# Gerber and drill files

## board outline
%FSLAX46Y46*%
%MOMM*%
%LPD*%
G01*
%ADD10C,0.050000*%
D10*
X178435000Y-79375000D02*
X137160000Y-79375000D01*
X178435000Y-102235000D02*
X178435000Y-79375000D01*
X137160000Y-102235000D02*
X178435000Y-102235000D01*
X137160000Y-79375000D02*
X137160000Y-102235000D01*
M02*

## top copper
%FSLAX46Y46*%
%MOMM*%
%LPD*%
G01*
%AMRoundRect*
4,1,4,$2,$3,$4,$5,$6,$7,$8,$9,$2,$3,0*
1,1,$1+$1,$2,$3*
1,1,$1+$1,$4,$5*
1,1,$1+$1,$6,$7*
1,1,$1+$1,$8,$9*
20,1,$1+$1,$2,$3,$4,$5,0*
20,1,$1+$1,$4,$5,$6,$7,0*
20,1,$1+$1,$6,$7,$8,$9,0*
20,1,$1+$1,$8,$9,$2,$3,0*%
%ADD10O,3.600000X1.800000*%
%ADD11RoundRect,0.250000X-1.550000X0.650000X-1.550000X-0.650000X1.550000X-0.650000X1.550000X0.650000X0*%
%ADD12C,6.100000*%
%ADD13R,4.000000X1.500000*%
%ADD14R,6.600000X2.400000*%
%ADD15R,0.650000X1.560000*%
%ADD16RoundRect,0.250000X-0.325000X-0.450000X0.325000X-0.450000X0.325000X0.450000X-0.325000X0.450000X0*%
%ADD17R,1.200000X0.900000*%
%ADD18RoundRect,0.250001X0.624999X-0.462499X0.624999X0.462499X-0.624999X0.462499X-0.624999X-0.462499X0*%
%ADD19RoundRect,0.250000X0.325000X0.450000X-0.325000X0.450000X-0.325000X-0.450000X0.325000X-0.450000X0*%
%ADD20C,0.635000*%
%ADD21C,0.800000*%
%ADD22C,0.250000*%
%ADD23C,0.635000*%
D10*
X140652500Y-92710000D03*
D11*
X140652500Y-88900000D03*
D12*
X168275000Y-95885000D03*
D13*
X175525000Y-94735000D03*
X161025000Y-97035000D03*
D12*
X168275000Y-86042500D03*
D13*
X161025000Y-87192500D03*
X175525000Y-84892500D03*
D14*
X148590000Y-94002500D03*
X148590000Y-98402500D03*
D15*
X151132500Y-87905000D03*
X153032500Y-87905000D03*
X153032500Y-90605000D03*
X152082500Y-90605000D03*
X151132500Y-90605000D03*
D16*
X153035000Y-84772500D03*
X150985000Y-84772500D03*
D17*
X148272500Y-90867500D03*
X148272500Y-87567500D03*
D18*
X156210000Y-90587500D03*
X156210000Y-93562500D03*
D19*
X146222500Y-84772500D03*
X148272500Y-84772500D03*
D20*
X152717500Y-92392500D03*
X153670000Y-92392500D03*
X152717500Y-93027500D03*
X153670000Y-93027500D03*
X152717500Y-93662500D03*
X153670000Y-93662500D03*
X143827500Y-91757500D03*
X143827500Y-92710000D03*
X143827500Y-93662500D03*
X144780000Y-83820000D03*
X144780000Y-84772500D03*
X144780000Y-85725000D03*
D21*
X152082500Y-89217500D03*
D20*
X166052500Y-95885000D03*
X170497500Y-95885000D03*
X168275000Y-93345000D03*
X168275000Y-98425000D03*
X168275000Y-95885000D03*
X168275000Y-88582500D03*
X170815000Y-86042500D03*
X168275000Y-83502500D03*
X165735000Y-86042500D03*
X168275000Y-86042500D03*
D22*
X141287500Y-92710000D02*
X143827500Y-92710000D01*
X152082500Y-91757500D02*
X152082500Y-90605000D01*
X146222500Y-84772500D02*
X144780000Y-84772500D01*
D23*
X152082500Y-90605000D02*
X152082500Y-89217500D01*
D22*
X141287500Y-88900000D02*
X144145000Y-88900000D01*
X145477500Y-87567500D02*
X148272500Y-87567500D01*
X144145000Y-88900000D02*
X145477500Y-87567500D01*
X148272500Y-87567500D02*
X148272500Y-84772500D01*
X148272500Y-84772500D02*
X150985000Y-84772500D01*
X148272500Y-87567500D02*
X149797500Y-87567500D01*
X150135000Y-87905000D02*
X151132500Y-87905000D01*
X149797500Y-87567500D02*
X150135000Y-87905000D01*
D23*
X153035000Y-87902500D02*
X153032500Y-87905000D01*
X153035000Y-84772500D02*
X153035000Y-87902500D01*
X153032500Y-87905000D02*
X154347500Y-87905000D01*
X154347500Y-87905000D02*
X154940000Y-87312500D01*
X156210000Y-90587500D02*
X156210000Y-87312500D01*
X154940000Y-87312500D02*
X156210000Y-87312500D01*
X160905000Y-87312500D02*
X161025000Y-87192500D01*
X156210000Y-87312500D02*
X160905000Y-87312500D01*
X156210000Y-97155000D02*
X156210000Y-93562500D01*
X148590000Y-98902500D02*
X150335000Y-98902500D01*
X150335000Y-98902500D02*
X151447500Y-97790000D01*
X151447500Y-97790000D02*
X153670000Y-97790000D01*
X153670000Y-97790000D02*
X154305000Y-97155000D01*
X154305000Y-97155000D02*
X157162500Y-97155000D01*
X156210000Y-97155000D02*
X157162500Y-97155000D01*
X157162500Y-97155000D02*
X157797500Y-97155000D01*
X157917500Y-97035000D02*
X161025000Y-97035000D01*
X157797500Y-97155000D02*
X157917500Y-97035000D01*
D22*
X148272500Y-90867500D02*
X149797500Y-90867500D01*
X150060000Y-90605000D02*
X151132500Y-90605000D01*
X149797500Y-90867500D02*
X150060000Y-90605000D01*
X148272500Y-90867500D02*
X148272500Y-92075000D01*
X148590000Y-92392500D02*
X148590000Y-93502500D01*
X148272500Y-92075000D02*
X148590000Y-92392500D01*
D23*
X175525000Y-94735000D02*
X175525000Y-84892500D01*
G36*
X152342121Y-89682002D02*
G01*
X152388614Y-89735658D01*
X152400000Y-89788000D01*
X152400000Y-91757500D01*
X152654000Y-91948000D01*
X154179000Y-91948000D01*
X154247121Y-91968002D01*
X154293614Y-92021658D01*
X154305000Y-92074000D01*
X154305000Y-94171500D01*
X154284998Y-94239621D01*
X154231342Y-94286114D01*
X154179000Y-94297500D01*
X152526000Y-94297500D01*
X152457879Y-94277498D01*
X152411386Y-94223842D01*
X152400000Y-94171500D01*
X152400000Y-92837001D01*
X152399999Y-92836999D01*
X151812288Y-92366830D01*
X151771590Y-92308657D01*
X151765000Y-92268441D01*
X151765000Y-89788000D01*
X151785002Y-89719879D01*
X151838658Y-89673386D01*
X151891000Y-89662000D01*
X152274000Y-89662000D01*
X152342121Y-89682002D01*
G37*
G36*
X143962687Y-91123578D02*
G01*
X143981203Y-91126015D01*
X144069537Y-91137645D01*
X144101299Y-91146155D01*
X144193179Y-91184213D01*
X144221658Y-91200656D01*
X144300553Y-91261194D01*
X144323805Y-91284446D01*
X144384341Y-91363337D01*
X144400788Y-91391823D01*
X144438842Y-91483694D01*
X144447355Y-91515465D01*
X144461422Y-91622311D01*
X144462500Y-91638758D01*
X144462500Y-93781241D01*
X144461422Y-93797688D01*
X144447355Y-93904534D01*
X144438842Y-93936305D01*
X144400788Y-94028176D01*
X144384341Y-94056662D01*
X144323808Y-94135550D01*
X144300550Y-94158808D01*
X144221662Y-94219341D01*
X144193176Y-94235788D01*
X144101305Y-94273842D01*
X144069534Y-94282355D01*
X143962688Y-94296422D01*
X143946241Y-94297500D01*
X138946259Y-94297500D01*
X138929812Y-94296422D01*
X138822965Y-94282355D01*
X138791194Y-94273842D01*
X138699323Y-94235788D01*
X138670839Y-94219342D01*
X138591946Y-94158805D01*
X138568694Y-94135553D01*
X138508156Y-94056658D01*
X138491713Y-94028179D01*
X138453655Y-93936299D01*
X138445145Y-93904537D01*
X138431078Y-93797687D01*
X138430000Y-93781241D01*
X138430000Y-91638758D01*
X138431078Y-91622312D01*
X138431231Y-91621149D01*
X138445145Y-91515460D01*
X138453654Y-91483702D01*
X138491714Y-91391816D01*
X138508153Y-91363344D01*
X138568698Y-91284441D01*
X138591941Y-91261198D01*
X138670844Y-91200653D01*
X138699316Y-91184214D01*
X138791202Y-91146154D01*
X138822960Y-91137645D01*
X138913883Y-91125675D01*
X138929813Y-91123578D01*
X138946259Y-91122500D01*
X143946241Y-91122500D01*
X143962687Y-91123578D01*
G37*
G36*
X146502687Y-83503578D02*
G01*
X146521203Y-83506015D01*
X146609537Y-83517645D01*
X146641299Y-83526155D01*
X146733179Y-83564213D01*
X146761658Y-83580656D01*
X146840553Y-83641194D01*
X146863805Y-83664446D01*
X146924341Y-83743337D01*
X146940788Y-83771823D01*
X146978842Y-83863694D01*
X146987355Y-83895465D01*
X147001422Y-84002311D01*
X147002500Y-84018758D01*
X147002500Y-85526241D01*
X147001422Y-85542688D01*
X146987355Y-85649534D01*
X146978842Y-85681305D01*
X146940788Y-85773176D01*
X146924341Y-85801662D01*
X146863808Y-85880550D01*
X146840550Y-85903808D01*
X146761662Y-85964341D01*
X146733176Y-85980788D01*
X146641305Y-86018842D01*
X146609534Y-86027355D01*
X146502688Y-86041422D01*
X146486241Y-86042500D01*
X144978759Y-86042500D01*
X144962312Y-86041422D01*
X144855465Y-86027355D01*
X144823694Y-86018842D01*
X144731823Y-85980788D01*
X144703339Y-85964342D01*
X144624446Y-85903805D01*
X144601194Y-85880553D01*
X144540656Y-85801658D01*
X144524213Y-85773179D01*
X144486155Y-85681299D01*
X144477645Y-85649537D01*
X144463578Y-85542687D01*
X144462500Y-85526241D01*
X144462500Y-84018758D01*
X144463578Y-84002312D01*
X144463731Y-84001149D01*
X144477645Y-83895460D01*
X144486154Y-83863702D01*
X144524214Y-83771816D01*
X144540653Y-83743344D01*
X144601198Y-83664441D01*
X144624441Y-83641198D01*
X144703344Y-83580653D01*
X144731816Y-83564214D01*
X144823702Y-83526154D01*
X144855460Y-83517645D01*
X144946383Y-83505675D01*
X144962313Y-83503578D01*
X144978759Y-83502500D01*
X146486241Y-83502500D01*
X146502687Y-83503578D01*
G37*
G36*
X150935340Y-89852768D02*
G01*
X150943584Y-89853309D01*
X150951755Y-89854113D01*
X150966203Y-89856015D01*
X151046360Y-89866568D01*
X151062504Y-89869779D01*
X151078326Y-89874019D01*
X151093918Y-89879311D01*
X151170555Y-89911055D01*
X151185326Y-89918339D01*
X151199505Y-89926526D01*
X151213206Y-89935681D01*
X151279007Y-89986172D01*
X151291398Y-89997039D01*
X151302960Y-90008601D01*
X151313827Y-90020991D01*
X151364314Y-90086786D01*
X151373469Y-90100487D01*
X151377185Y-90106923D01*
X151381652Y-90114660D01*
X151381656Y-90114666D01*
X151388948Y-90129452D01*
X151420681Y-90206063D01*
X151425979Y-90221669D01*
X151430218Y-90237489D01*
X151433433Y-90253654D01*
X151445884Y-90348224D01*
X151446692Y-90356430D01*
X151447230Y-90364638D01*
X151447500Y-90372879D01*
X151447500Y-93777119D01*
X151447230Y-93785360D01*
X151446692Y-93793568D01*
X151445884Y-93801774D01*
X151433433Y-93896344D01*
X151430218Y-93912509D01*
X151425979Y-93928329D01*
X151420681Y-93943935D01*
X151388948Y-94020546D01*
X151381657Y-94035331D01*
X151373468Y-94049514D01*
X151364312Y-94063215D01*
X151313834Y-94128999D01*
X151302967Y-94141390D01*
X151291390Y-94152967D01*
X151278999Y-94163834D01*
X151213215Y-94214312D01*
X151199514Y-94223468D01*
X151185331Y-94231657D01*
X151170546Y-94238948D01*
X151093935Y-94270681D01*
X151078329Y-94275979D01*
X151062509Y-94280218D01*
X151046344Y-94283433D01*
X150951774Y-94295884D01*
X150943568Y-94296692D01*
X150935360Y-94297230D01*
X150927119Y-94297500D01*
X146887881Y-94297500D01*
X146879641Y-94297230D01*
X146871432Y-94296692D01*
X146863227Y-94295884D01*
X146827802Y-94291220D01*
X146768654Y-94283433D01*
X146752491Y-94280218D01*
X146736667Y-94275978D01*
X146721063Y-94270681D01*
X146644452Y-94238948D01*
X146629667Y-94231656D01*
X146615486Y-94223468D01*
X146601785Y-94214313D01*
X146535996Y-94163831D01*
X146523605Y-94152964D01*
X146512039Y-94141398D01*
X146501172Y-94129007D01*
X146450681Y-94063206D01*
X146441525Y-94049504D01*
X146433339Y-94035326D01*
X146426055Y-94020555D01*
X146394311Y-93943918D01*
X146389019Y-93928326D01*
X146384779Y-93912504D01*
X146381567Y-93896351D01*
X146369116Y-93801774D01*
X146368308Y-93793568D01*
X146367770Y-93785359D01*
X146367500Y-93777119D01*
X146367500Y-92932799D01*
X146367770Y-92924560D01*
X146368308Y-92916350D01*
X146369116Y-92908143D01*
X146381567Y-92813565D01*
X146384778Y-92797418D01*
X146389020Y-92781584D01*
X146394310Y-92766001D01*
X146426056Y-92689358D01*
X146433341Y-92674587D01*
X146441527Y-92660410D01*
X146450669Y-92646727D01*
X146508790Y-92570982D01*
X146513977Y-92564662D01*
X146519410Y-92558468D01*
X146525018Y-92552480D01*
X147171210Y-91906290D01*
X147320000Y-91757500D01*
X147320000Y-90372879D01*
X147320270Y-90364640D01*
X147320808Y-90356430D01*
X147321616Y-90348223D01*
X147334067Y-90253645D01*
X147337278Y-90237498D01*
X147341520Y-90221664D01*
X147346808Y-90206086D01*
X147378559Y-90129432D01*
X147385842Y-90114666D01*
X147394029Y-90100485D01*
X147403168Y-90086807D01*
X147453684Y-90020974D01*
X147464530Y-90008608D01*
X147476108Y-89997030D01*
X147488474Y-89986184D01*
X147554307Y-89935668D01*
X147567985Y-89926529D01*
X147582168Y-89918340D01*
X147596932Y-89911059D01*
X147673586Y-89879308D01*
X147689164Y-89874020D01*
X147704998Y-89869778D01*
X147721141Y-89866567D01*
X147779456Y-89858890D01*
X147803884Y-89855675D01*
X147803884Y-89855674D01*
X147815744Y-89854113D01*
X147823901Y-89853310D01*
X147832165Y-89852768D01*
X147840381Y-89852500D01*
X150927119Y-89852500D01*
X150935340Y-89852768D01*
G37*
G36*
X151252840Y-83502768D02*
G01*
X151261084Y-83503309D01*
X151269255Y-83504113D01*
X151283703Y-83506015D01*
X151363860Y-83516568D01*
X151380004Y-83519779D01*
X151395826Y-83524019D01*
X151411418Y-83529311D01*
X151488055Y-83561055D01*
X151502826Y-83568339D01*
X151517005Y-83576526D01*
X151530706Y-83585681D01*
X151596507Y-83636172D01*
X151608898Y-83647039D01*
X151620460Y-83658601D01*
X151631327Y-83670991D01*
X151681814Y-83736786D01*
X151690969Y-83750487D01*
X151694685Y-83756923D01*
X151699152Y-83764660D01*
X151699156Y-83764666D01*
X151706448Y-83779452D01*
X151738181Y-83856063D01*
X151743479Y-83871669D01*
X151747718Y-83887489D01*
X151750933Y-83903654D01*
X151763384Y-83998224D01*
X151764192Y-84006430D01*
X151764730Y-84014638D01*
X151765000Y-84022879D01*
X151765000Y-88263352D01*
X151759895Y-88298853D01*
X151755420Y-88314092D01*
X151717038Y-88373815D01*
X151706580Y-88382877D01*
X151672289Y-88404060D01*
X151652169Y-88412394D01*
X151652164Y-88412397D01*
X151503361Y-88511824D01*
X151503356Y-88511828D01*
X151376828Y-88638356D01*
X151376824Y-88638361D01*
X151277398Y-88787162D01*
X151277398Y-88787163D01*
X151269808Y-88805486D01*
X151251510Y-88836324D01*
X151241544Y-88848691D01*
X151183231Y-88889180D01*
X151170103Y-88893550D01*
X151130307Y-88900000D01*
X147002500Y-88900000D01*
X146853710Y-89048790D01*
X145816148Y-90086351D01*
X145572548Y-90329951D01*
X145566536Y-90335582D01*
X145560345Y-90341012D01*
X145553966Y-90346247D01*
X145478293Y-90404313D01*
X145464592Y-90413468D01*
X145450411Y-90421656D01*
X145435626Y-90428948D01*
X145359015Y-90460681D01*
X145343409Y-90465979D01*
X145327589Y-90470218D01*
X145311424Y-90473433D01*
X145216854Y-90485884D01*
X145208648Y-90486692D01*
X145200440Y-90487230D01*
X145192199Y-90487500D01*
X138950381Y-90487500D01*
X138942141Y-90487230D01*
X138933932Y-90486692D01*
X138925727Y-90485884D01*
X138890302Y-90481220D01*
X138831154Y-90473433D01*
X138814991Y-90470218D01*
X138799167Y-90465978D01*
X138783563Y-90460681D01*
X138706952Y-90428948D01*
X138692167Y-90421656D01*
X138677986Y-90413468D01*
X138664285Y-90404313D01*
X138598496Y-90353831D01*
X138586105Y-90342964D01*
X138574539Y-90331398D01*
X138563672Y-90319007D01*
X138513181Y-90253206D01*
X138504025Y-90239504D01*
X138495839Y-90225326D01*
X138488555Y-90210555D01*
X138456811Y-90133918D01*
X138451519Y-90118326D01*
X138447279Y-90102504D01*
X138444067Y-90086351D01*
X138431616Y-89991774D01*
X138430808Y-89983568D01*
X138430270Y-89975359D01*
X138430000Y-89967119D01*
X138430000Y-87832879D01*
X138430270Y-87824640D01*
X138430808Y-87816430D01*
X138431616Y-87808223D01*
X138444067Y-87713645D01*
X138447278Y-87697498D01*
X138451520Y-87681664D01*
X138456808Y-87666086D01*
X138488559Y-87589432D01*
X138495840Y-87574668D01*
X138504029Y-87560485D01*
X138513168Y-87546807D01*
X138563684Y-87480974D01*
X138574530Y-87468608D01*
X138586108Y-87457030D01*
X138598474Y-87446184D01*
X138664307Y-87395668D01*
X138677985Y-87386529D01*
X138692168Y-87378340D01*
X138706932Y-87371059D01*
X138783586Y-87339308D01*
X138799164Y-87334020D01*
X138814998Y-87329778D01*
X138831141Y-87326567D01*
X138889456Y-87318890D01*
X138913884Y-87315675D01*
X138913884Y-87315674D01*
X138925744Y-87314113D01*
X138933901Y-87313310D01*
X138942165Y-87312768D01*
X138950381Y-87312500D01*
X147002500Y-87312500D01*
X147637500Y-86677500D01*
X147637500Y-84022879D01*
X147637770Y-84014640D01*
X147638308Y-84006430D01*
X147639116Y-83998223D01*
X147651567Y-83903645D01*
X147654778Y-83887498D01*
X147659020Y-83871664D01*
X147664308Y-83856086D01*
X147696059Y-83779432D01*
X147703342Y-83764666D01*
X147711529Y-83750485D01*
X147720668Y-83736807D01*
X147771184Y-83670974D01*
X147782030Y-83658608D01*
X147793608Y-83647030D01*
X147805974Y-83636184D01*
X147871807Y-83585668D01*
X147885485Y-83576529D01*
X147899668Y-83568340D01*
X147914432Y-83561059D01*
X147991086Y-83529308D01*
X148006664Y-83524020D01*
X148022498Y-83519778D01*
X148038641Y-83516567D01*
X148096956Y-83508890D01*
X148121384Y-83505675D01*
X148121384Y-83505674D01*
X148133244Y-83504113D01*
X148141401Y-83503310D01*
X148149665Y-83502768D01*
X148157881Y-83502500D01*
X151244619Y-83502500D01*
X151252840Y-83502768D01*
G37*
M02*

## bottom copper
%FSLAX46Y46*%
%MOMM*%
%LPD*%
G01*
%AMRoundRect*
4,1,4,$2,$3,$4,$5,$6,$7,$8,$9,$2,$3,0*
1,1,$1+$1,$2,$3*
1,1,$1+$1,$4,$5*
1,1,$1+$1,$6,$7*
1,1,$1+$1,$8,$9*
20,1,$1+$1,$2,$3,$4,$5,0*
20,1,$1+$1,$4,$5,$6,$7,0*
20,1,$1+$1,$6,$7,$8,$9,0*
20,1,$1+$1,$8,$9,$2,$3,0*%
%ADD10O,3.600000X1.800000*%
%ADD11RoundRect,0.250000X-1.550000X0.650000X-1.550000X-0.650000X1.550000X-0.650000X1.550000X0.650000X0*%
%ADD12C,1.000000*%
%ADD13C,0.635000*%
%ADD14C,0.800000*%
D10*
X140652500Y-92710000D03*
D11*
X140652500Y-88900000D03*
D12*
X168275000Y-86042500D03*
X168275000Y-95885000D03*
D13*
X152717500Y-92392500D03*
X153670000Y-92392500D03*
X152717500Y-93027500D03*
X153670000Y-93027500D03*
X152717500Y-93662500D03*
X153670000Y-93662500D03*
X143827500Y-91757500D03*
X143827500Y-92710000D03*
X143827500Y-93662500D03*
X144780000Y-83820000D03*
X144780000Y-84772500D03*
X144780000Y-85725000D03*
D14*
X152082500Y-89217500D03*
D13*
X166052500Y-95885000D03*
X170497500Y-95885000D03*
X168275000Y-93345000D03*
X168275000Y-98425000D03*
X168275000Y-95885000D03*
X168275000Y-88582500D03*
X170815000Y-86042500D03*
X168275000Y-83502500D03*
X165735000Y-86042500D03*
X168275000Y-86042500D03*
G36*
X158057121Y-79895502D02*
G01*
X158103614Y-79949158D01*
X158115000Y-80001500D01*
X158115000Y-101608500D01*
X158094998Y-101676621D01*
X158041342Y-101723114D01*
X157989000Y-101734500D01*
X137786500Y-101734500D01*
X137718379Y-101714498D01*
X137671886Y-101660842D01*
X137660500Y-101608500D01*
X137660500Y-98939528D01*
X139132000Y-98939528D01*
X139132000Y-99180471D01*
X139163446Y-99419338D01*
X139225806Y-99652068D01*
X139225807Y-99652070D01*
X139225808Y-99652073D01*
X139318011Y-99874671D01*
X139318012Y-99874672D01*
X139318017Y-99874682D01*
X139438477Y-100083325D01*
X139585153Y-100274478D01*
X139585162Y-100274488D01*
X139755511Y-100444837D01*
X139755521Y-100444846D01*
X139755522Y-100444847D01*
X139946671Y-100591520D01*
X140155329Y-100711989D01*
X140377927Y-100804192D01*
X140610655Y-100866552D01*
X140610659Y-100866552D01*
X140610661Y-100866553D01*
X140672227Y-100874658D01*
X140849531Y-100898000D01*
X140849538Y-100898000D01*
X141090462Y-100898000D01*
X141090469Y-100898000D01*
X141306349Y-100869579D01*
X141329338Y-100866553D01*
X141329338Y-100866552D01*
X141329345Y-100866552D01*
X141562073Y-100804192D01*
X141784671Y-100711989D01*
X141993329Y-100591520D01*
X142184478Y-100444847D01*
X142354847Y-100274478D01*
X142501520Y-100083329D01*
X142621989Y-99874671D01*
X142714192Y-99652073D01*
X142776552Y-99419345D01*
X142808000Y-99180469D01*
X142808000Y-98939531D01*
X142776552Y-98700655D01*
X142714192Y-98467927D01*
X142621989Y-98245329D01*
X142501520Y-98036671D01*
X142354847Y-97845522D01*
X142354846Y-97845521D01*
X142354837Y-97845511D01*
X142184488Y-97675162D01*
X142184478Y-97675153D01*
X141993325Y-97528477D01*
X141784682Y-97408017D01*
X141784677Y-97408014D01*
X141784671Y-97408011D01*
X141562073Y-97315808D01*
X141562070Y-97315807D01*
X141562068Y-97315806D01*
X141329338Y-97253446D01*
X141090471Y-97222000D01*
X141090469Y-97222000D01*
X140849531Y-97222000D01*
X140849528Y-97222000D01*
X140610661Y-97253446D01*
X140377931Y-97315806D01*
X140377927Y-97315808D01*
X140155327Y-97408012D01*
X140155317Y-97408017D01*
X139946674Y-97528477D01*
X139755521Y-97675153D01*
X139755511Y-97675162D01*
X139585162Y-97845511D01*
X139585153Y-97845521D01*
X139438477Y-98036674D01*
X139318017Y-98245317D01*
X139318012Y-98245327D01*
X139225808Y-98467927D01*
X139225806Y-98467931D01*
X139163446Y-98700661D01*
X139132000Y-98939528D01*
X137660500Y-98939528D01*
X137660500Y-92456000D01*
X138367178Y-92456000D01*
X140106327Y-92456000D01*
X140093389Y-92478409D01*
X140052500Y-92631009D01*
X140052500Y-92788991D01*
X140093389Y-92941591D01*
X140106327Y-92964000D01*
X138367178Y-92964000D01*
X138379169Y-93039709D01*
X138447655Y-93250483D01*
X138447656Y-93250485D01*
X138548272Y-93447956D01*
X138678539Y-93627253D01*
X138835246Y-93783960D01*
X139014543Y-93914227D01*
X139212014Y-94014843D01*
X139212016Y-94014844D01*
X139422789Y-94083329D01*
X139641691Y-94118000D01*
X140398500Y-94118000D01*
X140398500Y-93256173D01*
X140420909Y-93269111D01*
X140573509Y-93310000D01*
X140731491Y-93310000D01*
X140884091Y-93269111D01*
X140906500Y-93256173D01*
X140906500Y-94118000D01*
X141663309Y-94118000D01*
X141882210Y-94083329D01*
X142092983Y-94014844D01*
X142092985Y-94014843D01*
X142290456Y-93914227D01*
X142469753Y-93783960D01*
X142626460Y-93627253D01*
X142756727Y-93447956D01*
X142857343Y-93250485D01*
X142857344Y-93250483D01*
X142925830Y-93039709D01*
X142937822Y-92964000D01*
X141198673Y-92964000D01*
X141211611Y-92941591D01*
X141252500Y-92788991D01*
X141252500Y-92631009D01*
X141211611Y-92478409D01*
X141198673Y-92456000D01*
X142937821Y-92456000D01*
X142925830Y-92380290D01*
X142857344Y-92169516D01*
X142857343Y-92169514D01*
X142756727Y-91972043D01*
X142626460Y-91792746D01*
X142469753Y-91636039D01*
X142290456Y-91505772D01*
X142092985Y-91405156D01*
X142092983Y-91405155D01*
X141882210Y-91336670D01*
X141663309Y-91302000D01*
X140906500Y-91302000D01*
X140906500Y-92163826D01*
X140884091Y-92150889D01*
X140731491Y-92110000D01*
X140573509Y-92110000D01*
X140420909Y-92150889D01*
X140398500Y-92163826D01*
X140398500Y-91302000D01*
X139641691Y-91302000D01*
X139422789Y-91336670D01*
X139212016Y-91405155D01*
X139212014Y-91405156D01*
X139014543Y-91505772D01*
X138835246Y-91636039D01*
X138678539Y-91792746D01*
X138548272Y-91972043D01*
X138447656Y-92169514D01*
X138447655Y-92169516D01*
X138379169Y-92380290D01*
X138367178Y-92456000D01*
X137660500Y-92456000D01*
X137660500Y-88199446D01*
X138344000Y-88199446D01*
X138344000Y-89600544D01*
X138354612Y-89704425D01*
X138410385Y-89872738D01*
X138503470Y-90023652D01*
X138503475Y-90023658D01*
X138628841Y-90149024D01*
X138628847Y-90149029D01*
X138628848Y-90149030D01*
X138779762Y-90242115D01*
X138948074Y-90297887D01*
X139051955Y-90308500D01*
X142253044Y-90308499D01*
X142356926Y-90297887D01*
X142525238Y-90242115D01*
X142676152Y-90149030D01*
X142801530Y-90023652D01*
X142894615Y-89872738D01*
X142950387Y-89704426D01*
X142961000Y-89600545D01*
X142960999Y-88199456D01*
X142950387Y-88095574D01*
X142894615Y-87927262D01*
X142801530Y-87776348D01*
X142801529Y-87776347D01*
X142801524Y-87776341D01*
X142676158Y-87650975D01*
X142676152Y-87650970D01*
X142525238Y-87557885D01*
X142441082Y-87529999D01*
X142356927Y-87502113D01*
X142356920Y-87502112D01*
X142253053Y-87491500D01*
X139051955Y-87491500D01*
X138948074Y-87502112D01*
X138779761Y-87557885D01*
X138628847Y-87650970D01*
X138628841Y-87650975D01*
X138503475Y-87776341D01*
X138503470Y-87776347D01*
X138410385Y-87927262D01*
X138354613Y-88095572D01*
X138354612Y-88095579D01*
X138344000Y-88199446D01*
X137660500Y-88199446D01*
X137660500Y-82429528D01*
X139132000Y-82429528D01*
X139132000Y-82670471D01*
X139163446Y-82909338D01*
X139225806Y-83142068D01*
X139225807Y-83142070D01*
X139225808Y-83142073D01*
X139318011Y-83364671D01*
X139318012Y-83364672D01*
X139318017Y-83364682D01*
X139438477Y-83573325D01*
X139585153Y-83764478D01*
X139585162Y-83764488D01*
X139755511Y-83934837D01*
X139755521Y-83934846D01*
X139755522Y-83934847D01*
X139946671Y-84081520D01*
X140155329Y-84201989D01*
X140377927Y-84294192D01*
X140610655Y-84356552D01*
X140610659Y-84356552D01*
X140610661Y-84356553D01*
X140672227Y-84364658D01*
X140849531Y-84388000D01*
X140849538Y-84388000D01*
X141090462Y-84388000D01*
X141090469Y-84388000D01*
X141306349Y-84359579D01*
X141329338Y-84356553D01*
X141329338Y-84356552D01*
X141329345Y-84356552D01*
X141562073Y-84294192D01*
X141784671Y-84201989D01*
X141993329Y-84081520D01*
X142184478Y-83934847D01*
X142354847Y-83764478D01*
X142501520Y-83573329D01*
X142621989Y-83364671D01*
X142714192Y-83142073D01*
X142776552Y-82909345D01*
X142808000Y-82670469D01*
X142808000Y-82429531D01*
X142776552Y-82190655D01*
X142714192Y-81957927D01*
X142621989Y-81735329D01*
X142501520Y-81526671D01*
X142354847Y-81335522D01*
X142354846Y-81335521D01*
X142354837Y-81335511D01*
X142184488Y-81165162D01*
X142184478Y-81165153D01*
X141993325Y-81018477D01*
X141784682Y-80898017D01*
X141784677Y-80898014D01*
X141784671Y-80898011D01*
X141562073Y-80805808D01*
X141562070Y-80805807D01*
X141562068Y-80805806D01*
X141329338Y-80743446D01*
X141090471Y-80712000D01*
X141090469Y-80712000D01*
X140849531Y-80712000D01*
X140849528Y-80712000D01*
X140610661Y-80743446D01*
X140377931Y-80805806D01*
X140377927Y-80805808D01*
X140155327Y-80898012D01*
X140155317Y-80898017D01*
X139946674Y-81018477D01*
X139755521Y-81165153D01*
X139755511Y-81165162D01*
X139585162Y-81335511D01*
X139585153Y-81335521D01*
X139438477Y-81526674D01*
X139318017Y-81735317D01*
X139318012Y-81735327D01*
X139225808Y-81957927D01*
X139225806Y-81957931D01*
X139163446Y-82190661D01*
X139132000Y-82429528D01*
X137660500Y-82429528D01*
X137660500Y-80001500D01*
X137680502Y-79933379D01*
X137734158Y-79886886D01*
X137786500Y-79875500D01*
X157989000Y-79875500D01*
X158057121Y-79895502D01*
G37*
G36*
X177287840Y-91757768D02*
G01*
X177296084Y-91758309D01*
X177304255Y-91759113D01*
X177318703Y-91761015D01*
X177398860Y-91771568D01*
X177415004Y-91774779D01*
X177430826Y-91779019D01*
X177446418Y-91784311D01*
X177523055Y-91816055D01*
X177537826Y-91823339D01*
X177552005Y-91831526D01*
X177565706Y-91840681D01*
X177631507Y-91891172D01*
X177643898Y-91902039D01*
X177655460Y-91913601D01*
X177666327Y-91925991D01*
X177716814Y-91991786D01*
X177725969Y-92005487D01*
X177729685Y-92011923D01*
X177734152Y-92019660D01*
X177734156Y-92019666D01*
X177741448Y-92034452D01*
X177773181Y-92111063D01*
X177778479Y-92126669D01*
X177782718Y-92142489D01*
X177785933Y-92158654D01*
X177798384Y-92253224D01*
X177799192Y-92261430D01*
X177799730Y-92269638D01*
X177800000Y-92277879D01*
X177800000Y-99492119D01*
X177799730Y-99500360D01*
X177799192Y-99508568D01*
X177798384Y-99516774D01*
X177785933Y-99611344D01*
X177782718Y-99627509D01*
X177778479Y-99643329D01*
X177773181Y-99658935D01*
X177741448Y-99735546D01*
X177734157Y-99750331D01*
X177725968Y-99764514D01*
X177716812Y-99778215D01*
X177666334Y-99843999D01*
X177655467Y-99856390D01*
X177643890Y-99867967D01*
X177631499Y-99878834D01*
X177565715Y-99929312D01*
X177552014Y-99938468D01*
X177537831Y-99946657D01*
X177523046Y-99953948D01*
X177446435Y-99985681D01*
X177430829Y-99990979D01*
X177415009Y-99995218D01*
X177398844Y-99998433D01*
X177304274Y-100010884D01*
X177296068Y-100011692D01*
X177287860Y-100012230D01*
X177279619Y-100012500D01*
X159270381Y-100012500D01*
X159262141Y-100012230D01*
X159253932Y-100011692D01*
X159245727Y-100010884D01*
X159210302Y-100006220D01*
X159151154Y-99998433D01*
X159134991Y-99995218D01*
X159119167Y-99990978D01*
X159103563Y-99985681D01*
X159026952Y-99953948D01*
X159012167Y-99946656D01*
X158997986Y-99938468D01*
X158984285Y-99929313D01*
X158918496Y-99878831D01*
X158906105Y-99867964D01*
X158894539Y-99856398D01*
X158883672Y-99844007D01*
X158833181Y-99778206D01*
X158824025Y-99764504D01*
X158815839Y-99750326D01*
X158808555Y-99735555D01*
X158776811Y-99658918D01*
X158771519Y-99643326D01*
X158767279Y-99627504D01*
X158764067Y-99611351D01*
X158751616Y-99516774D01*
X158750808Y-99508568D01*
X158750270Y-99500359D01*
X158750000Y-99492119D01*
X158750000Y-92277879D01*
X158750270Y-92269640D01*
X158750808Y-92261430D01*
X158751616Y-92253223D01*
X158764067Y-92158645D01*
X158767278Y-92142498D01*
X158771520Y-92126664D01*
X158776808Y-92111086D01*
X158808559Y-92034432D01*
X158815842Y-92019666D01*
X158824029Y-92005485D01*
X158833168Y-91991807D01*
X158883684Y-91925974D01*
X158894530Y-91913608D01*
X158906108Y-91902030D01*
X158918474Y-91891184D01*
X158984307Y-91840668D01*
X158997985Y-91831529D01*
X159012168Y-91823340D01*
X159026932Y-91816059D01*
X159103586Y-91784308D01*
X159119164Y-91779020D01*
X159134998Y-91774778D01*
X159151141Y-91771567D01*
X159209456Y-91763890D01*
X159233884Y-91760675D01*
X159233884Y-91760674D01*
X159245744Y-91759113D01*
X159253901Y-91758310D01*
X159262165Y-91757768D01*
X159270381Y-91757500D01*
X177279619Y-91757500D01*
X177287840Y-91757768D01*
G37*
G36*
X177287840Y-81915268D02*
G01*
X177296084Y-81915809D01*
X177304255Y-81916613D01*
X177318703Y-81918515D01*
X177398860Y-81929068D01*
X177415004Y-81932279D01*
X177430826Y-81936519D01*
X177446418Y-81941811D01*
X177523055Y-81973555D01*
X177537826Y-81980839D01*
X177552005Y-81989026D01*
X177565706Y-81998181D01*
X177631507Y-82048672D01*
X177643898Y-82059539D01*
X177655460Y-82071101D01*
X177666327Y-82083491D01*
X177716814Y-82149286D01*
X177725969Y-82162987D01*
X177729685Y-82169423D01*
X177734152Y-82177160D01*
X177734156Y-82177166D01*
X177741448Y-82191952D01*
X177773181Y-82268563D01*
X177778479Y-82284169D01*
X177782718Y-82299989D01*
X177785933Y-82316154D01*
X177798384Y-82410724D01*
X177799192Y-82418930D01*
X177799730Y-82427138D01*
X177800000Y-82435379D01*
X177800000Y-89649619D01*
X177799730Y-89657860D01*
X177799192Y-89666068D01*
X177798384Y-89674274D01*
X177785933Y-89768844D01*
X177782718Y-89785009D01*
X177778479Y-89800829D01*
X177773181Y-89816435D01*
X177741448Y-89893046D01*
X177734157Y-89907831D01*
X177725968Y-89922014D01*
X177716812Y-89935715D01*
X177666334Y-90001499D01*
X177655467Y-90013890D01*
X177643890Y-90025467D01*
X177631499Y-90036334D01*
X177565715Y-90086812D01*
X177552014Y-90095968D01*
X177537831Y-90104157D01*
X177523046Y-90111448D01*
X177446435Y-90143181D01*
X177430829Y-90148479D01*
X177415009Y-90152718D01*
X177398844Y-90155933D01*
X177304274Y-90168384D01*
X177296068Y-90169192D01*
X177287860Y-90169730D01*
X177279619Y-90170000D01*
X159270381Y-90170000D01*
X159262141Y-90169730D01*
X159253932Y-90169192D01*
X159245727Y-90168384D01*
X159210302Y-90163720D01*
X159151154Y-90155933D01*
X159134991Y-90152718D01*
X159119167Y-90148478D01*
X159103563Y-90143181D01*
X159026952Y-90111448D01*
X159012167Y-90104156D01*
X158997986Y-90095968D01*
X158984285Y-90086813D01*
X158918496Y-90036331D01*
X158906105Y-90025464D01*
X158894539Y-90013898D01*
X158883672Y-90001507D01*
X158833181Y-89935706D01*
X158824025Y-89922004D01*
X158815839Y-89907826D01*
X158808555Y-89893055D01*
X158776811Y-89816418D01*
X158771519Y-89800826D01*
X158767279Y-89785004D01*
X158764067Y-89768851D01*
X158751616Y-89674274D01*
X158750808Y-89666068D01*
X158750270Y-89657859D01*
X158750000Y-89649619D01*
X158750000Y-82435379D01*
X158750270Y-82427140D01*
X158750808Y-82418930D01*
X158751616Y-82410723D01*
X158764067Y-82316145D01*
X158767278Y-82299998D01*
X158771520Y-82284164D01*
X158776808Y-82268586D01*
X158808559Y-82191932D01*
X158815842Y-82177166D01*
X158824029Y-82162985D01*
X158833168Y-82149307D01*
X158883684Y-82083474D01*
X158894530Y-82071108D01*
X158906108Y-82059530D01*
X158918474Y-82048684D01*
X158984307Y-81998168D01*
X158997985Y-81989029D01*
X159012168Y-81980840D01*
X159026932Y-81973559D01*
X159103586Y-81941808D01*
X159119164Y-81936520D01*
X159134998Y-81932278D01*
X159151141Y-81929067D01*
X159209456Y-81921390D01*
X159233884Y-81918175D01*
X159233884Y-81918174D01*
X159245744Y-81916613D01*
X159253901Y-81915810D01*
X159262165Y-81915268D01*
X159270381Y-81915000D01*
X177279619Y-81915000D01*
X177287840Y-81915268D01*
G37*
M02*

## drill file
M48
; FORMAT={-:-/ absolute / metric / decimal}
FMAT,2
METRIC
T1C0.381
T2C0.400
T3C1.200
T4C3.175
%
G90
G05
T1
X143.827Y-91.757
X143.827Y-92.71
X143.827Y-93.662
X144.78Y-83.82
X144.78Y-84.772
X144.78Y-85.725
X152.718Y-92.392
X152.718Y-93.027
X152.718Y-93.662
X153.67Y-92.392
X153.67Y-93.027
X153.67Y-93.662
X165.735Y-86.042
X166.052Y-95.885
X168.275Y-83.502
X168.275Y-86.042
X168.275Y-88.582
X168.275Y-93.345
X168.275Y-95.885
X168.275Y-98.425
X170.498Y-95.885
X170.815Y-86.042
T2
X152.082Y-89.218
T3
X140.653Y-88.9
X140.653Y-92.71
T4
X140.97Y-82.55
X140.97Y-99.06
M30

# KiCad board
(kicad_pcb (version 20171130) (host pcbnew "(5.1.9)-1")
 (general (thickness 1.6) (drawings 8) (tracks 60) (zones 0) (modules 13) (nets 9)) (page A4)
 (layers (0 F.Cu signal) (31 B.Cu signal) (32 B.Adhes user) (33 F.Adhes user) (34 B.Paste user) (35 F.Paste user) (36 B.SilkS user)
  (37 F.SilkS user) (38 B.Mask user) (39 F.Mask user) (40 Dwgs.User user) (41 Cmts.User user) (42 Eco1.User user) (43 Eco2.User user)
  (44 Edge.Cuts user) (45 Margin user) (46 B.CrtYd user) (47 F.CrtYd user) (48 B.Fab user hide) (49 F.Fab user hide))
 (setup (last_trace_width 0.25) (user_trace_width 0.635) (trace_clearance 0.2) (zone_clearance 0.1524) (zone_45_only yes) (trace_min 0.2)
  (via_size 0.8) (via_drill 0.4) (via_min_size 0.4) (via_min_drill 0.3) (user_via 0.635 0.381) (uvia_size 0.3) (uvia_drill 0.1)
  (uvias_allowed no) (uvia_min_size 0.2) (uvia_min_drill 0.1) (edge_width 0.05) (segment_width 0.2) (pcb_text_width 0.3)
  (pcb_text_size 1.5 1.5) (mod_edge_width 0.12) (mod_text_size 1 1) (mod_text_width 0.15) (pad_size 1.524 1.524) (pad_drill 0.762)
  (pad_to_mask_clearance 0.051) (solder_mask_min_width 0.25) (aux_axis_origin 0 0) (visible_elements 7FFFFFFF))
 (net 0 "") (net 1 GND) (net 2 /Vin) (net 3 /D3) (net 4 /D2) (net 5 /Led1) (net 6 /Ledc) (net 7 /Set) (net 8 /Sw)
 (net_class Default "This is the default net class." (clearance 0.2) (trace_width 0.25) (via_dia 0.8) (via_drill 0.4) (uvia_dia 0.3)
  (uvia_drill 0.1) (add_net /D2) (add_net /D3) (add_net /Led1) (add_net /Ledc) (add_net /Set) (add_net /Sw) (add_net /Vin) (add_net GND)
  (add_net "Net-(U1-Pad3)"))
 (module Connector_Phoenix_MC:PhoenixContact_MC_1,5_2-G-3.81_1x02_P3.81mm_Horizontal (layer F.Cu) (at 140.6525 88.9 270)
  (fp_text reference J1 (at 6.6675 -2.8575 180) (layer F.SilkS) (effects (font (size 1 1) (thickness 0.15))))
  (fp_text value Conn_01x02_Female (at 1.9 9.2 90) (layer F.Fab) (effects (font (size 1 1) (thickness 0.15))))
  (pad 2 thru_hole oval (at 3.81 0 270) (size 1.8 3.6) (drill 1.2) (layers *.Cu *.Mask) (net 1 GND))
  (pad 1 thru_hole roundrect (at 0 0 270) (size 1.8 3.6) (drill 1.2) (layers *.Cu *.Mask) (roundrect_rratio 0.138889) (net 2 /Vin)))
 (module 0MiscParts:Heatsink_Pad (layer B.Cu) (at 168.275 86.0425)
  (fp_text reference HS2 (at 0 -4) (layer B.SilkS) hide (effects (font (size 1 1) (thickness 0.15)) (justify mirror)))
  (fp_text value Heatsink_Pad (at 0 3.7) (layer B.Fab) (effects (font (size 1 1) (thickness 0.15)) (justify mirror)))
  (pad 1 smd circle (at 0 0) (size 1 1) (layers B.Cu B.Paste B.Mask) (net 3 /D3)))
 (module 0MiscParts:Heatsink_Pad (layer B.Cu) (at 168.275 95.885)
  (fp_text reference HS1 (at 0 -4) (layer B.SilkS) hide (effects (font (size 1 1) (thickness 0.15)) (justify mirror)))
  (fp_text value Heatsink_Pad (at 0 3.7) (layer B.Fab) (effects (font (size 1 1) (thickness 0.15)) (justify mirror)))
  (pad 1 smd circle (at 0 0) (size 1 1) (layers B.Cu B.Paste B.Mask) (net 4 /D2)))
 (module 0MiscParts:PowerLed (layer F.Cu) (at 168.275 95.885)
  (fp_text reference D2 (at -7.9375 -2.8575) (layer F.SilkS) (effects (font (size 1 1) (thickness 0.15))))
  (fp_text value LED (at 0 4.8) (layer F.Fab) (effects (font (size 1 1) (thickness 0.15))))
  (pad 3 smd circle (at 0 0) (size 6.1 6.1) (layers F.Cu F.Paste F.Mask) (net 4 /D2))
  (pad 2 smd rect (at 7.25 -1.15) (size 4 1.5) (layers F.Cu F.Paste F.Mask) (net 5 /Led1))
  (pad 1 smd rect (at -7.25 1.15) (size 4 1.5) (layers F.Cu F.Paste F.Mask) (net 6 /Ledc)))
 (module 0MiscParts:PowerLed (layer F.Cu) (at 168.275 86.0425 180)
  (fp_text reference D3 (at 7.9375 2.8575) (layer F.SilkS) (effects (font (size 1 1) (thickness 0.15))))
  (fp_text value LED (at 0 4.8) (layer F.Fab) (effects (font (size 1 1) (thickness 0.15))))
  (pad 3 smd circle (at 0 0 180) (size 6.1 6.1) (layers F.Cu F.Paste F.Mask) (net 3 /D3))
  (pad 2 smd rect (at 7.25 -1.15 180) (size 4 1.5) (layers F.Cu F.Paste F.Mask) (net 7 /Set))
  (pad 1 smd rect (at -7.25 1.15 180) (size 4 1.5) (layers F.Cu F.Paste F.Mask) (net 5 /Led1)))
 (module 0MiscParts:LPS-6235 (layer F.Cu) (at 148.59 96.2025 90)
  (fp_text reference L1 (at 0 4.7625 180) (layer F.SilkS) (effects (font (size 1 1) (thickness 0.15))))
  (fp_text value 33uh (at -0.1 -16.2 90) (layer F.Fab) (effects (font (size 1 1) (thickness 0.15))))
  (pad 2 smd rect (at 2.2 0 90) (size 2.4 6.6) (layers F.Cu F.Paste F.Mask) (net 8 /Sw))
  (pad 1 smd rect (at -2.2 0 90) (size 2.4 6.6) (layers F.Cu F.Paste F.Mask) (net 6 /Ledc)))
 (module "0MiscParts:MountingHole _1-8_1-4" (layer F.Cu) (at 140.97 99.06)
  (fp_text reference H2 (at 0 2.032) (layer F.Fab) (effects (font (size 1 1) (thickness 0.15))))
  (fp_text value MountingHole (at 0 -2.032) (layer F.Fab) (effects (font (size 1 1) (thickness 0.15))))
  (pad "" np_thru_hole circle (at 0 0) (size 3.175 3.175) (drill 3.175) (layers *.Cu *.Mask)))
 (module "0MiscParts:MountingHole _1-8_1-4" (layer F.Cu) (at 140.97 82.55)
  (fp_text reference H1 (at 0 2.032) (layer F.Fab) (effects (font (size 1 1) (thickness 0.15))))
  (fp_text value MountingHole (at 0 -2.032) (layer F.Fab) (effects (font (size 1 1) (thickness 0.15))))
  (pad "" np_thru_hole circle (at 0 0) (size 3.175 3.175) (drill 3.175) (layers *.Cu *.Mask)))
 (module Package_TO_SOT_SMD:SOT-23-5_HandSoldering (layer F.Cu) (at 152.0825 89.255 90)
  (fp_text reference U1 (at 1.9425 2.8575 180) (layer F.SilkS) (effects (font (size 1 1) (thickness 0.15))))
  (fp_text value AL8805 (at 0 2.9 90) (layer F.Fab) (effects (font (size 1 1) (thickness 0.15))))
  (pad 5 smd rect (at 1.35 -0.95 90) (size 1.56 0.65) (layers F.Cu F.Paste F.Mask) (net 2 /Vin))
  (pad 4 smd rect (at 1.35 0.95 90) (size 1.56 0.65) (layers F.Cu F.Paste F.Mask) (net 7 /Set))
  (pad 3 smd rect (at -1.35 0.95 90) (size 1.56 0.65) (layers F.Cu F.Paste F.Mask))
  (pad 2 smd rect (at -1.35 0 90) (size 1.56 0.65) (layers F.Cu F.Paste F.Mask) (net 1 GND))
  (pad 1 smd rect (at -1.35 -0.95 90) (size 1.56 0.65) (layers F.Cu F.Paste F.Mask) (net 8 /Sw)))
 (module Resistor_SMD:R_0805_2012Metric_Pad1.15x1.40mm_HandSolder (layer F.Cu) (at 152.01 84.7725)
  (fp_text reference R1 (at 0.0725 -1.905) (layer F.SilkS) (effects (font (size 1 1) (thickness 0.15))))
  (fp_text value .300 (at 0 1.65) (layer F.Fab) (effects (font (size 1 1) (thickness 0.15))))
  (pad 2 smd roundrect (at 1.025 0) (size 1.15 1.4) (layers F.Cu F.Paste F.Mask) (roundrect_rratio 0.217391) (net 7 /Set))
  (pad 1 smd roundrect (at -1.025 0) (size 1.15 1.4) (layers F.Cu F.Paste F.Mask) (roundrect_rratio 0.217391) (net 2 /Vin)))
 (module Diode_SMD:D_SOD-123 (layer F.Cu) (at 148.2725 89.2175 270)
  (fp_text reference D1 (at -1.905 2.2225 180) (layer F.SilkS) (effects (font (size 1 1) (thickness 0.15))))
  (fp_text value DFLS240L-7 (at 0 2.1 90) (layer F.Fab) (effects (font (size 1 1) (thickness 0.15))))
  (pad 2 smd rect (at 1.65 0 270) (size 0.9 1.2) (layers F.Cu F.Paste F.Mask) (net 8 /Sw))
  (pad 1 smd rect (at -1.65 0 270) (size 0.9 1.2) (layers F.Cu F.Paste F.Mask) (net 2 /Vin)))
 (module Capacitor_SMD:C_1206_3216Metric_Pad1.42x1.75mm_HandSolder (layer F.Cu) (at 156.21 92.075 90)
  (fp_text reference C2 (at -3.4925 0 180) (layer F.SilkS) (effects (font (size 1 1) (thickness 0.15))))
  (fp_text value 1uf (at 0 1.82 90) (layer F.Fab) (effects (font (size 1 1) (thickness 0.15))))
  (pad 2 smd roundrect (at 1.4875 0 90) (size 1.425 1.75) (layers F.Cu F.Paste F.Mask) (roundrect_rratio 0.175439) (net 7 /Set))
  (pad 1 smd roundrect (at -1.4875 0 90) (size 1.425 1.75) (layers F.Cu F.Paste F.Mask) (roundrect_rratio 0.175439) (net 6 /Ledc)))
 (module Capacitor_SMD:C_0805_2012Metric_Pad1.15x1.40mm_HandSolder (layer F.Cu) (at 147.2475 84.7725 180)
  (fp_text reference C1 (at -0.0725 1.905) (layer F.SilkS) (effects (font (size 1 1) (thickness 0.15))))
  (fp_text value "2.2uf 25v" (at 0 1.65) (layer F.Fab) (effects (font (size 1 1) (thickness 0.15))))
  (pad 2 smd roundrect (at 1.025 0 180) (size 1.15 1.4) (layers F.Cu F.Paste F.Mask) (roundrect_rratio 0.217391) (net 1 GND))
  (pad 1 smd roundrect (at -1.025 0 180) (size 1.15 1.4) (layers F.Cu F.Paste F.Mask) (roundrect_rratio 0.217391) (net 2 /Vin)))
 (gr_line (start 178.435 79.375) (end 137.16 79.375) (layer Edge.Cuts) (width 0.05))
 (gr_line (start 178.435 102.235) (end 178.435 79.375) (layer Edge.Cuts) (width 0.05))
 (gr_line (start 137.16 102.235) (end 178.435 102.235) (layer Edge.Cuts) (width 0.05))
 (gr_line (start 137.16 79.375) (end 137.16 102.235) (layer Edge.Cuts) (width 0.05))
 (via (at 152.7175 92.3925) (size 0.635) (drill 0.381) (layers F.Cu B.Cu) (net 1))
 (via (at 153.67 92.3925) (size 0.635) (drill 0.381) (layers F.Cu B.Cu) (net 1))
 (via (at 152.7175 93.0275) (size 0.635) (drill 0.381) (layers F.Cu B.Cu) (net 1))
 (via (at 153.67 93.0275) (size 0.635) (drill 0.381) (layers F.Cu B.Cu) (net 1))
 (via (at 152.7175 93.6625) (size 0.635) (drill 0.381) (layers F.Cu B.Cu) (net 1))
 (via (at 153.67 93.6625) (size 0.635) (drill 0.381) (layers F.Cu B.Cu) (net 1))
 (via (at 143.8275 91.7575) (size 0.635) (drill 0.381) (layers F.Cu B.Cu) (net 1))
 (via (at 143.8275 92.71) (size 0.635) (drill 0.381) (layers F.Cu B.Cu) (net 1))
 (via (at 143.8275 93.6625) (size 0.635) (drill 0.381) (layers F.Cu B.Cu) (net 1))
 (segment (start 141.2875 92.71) (end 143.8275 92.71) (width 0.25) (layer F.Cu) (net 1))
 (via (at 144.78 83.82) (size 0.635) (drill 0.381) (layers F.Cu B.Cu) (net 1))
 (via (at 144.78 84.7725) (size 0.635) (drill 0.381) (layers F.Cu B.Cu) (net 1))
 (via (at 144.78 85.725) (size 0.635) (drill 0.381) (layers F.Cu B.Cu) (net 1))
 (segment (start 152.0825 91.7575) (end 152.0825 90.605) (width 0.25) (layer F.Cu) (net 1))
 (segment (start 146.2225 84.7725) (end 144.78 84.7725) (width 0.25) (layer F.Cu) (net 1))
 (via (at 152.0825 89.2175) (size 0.8) (drill 0.4) (layers F.Cu B.Cu) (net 1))
 (segment (start 152.0825 90.605) (end 152.0825 89.2175) (width 0.635) (layer F.Cu) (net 1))
 (segment (start 141.2875 88.9) (end 144.145 88.9) (width 0.25) (layer F.Cu) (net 2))
 (segment (start 145.4775 87.5675) (end 148.2725 87.5675) (width 0.25) (layer F.Cu) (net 2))
 (segment (start 144.145 88.9) (end 145.4775 87.5675) (width 0.25) (layer F.Cu) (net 2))
 (segment (start 148.2725 87.5675) (end 148.2725 84.7725) (width 0.25) (layer F.Cu) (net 2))
 (segment (start 148.2725 84.7725) (end 150.985 84.7725) (width 0.25) (layer F.Cu) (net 2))
 (segment (start 148.2725 87.5675) (end 149.7975 87.5675) (width 0.25) (layer F.Cu) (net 2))
 (segment (start 150.135 87.905) (end 151.1325 87.905) (width 0.25) (layer F.Cu) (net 2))
 (segment (start 149.7975 87.5675) (end 150.135 87.905) (width 0.25) (layer F.Cu) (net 2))
 (segment (start 153.035 87.9025) (end 153.0325 87.905) (width 0.635) (layer F.Cu) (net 7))
 (segment (start 153.035 84.7725) (end 153.035 87.9025) (width 0.635) (layer F.Cu) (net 7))
 (segment (start 153.0325 87.905) (end 154.3475 87.905) (width 0.635) (layer F.Cu) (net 7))
 (segment (start 154.3475 87.905) (end 154.94 87.3125) (width 0.635) (layer F.Cu) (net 7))
 (segment (start 156.21 90.5875) (end 156.21 87.3125) (width 0.635) (layer F.Cu) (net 7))
 (segment (start 154.94 87.3125) (end 156.21 87.3125) (width 0.635) (layer F.Cu) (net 7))
 (segment (start 160.905 87.3125) (end 161.025 87.1925) (width 0.635) (layer F.Cu) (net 7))
 (segment (start 156.21 87.3125) (end 160.905 87.3125) (width 0.635) (layer F.Cu) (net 7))
 (segment (start 156.21 97.155) (end 156.21 93.5625) (width 0.635) (layer F.Cu) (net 6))
 (segment (start 148.59 98.9025) (end 150.335 98.9025) (width 0.635) (layer F.Cu) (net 6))
 (segment (start 150.335 98.9025) (end 151.4475 97.79) (width 0.635) (layer F.Cu) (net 6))
 (segment (start 151.4475 97.79) (end 153.67 97.79) (width 0.635) (layer F.Cu) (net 6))
 (segment (start 153.67 97.79) (end 154.305 97.155) (width 0.635) (layer F.Cu) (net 6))
 (segment (start 154.305 97.155) (end 157.1625 97.155) (width 0.635) (layer F.Cu) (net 6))
 (segment (start 156.21 97.155) (end 157.1625 97.155) (width 0.635) (layer F.Cu) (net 6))
 (segment (start 157.1625 97.155) (end 157.7975 97.155) (width 0.635) (layer F.Cu) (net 6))
 (segment (start 157.9175 97.035) (end 161.025 97.035) (width 0.635) (layer F.Cu) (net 6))
 (segment (start 157.7975 97.155) (end 157.9175 97.035) (width 0.635) (layer F.Cu) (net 6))
 (segment (start 148.2725 90.8675) (end 149.7975 90.8675) (width 0.25) (layer F.Cu) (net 8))
 (segment (start 150.06 90.605) (end 151.1325 90.605) (width 0.25) (layer F.Cu) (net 8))
 (segment (start 149.7975 90.8675) (end 150.06 90.605) (width 0.25) (layer F.Cu) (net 8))
 (segment (start 148.2725 90.8675) (end 148.2725 92.075) (width 0.25) (layer F.Cu) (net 8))
 (segment (start 148.59 92.3925) (end 148.59 93.5025) (width 0.25) (layer F.Cu) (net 8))
 (segment (start 148.2725 92.075) (end 148.59 92.3925) (width 0.25) (layer F.Cu) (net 8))
 (segment (start 175.525 94.735) (end 175.525 84.8925) (width 0.635) (layer F.Cu) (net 5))
 (via (at 166.0525 95.885) (size 0.635) (drill 0.381) (layers F.Cu B.Cu) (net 4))
 (via (at 170.4975 95.885) (size 0.635) (drill 0.381) (layers F.Cu B.Cu) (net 4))
 (via (at 168.275 93.345) (size 0.635) (drill 0.381) (layers F.Cu B.Cu) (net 4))
 (via (at 168.275 98.425) (size 0.635) (drill 0.381) (layers F.Cu B.Cu) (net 4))
 (via (at 168.275 95.885) (size 0.635) (drill 0.381) (layers F.Cu B.Cu) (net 4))
 (via (at 168.275 88.5825) (size 0.635) (drill 0.381) (layers F.Cu B.Cu) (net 3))
 (via (at 170.815 86.0425) (size 0.635) (drill 0.381) (layers F.Cu B.Cu) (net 3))
 (via (at 168.275 83.5025) (size 0.635) (drill 0.381) (layers F.Cu B.Cu) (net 3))
 (via (at 165.735 86.0425) (size 0.635) (drill 0.381) (layers F.Cu B.Cu) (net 3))
 (via (at 168.275 86.0425) (size 0.635) (drill 0.381) (layers F.Cu B.Cu) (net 3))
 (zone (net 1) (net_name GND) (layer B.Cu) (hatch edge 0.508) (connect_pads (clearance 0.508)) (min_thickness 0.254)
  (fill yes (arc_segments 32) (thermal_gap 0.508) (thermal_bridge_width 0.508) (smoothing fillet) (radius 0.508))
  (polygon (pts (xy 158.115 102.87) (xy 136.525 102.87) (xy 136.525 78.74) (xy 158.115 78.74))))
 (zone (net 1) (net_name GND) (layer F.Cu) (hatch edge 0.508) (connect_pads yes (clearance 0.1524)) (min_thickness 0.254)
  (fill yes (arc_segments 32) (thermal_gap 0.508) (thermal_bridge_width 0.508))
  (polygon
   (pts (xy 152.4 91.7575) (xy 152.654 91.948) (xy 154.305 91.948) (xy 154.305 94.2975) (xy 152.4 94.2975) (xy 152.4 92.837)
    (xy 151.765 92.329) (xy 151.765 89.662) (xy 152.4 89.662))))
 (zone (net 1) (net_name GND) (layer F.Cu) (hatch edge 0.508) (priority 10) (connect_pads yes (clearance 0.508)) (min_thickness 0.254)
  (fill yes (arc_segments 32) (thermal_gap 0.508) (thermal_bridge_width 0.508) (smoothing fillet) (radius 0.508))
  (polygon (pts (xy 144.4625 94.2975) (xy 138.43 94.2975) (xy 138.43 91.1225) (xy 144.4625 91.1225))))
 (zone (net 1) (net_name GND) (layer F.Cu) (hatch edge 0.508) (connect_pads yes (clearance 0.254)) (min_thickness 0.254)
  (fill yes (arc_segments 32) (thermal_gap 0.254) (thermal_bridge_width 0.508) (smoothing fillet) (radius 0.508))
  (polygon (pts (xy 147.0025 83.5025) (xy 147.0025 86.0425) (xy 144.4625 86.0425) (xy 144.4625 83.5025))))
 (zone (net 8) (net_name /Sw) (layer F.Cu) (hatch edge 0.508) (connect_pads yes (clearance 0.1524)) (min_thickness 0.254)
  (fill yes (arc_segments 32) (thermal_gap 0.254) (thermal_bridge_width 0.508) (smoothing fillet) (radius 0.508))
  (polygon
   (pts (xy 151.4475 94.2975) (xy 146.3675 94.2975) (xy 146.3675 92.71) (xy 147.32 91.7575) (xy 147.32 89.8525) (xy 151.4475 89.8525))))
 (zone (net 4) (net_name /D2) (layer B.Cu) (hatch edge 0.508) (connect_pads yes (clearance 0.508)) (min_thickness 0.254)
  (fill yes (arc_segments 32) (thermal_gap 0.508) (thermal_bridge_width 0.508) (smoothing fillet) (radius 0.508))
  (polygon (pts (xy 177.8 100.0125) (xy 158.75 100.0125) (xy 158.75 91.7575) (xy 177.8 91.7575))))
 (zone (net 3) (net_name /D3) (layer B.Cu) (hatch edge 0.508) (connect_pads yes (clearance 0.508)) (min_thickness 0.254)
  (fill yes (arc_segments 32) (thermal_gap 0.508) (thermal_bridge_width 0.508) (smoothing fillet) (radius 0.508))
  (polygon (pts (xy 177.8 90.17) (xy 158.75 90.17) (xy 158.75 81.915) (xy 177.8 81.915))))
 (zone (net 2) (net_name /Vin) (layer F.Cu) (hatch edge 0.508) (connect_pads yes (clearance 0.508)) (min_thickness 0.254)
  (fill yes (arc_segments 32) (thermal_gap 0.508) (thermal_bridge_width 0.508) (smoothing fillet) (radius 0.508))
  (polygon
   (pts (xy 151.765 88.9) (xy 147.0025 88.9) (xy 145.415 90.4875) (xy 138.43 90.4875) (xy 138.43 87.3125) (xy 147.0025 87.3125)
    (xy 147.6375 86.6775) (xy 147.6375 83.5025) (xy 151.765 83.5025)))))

